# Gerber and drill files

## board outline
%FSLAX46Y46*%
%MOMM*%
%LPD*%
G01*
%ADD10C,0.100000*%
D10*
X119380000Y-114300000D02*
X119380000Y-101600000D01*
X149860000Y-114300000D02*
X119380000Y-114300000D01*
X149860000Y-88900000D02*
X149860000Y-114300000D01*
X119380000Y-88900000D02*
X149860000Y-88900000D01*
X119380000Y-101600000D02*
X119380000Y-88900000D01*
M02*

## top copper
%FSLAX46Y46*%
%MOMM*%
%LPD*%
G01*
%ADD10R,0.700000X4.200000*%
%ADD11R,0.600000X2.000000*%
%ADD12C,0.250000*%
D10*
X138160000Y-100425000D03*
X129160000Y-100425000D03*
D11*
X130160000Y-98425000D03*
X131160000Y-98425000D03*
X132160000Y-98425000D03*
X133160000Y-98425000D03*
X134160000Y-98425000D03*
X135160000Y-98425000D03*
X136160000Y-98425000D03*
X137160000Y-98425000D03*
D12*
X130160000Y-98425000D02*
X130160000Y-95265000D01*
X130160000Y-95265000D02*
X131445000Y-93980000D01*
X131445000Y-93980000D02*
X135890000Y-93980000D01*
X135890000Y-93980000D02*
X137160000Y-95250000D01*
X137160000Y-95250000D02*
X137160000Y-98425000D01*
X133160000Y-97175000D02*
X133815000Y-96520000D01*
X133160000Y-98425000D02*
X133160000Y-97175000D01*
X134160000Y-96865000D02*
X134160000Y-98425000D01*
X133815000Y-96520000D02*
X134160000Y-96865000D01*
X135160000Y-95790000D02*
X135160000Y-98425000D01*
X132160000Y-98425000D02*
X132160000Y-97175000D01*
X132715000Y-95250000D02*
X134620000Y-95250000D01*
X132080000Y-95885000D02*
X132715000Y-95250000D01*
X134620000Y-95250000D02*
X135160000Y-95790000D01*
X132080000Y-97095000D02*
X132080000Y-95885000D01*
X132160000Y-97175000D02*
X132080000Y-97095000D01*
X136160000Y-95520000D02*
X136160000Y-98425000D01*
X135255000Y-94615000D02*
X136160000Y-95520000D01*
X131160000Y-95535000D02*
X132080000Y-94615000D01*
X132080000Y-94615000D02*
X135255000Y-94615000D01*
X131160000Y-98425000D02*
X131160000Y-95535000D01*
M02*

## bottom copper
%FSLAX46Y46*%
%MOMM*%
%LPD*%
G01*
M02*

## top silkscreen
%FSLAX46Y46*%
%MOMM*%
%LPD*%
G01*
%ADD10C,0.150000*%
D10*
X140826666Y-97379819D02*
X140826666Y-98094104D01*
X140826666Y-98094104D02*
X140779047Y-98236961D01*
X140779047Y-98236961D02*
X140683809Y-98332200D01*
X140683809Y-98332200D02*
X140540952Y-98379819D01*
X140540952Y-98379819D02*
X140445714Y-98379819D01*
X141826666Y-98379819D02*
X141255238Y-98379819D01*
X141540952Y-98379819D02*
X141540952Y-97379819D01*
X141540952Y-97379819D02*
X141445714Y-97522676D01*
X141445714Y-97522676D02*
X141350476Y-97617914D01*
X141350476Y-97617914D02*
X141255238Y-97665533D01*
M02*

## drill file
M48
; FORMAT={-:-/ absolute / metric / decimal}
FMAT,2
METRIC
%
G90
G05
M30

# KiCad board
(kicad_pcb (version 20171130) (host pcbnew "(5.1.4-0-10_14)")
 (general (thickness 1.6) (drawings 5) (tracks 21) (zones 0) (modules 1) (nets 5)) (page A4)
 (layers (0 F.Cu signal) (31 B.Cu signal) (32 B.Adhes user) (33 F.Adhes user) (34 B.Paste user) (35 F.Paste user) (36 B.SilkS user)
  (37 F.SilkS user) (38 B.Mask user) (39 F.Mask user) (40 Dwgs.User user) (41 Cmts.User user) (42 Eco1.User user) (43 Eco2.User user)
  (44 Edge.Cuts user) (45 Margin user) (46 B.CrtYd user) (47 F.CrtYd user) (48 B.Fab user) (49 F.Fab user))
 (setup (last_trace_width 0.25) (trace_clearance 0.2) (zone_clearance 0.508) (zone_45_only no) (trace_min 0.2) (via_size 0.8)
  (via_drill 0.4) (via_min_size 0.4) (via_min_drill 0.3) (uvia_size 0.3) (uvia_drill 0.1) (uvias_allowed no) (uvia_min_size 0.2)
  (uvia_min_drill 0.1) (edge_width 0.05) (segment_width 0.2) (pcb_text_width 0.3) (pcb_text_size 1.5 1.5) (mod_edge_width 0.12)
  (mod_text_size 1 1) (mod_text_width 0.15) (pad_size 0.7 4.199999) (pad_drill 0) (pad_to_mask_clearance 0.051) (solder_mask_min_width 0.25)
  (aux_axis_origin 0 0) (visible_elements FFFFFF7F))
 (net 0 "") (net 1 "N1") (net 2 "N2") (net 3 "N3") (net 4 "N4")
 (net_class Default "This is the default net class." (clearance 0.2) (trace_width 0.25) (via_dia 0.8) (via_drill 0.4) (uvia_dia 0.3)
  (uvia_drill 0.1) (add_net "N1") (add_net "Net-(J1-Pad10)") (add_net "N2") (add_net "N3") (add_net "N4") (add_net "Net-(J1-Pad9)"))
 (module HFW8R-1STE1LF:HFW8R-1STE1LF (layer F.Cu) (at 137.16 98.425)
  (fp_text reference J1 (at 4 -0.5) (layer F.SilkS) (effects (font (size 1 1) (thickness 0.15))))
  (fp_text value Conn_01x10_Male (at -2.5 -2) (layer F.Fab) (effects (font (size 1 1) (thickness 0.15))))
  (pad 10 smd rect (at 1 2) (size 0.7 4.2) (layers F.Cu F.Paste F.Mask))
  (pad 9 smd rect (at -8 2) (size 0.7 4.2) (layers F.Cu F.Paste F.Mask))
  (pad 8 smd rect (at -7 0) (size 0.6 2) (layers F.Cu F.Paste F.Mask) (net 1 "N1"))
  (pad 7 smd rect (at -6 0) (size 0.6 2) (layers F.Cu F.Paste F.Mask) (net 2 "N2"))
  (pad 6 smd rect (at -5 0) (size 0.6 2) (layers F.Cu F.Paste F.Mask) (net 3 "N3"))
  (pad 5 smd rect (at -4 0) (size 0.6 2) (layers F.Cu F.Paste F.Mask) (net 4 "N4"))
  (pad 4 smd rect (at -3 0) (size 0.6 2) (layers F.Cu F.Paste F.Mask) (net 4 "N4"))
  (pad 3 smd rect (at -2 0) (size 0.6 2) (layers F.Cu F.Paste F.Mask) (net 3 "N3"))
  (pad 2 smd rect (at -1 0) (size 0.6 2) (layers F.Cu F.Paste F.Mask) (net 2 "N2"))
  (pad 1 smd rect (at 0 0) (size 0.6 2) (layers F.Cu F.Paste F.Mask) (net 1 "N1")))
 (gr_line (start 119.38 114.3) (end 119.38 101.6) (layer Edge.Cuts) (width 0.1))
 (gr_line (start 149.86 114.3) (end 119.38 114.3) (layer Edge.Cuts) (width 0.1))
 (gr_line (start 149.86 88.9) (end 149.86 114.3) (layer Edge.Cuts) (width 0.1))
 (gr_line (start 119.38 88.9) (end 149.86 88.9) (layer Edge.Cuts) (width 0.1))
 (gr_line (start 119.38 101.6) (end 119.38 88.9) (layer Edge.Cuts) (width 0.1))
 (segment (start 130.16 98.425) (end 130.16 95.265) (width 0.25) (layer F.Cu) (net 1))
 (segment (start 130.16 95.265) (end 131.445 93.98) (width 0.25) (layer F.Cu) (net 1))
 (segment (start 131.445 93.98) (end 135.89 93.98) (width 0.25) (layer F.Cu) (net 1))
 (segment (start 135.89 93.98) (end 137.16 95.25) (width 0.25) (layer F.Cu) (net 1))
 (segment (start 137.16 95.25) (end 137.16 98.425) (width 0.25) (layer F.Cu) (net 1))
 (segment (start 133.16 97.175) (end 133.815 96.52) (width 0.25) (layer F.Cu) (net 4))
 (segment (start 133.16 98.425) (end 133.16 97.175) (width 0.25) (layer F.Cu) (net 4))
 (segment (start 134.16 96.865) (end 134.16 98.425) (width 0.25) (layer F.Cu) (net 4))
 (segment (start 133.815 96.52) (end 134.16 96.865) (width 0.25) (layer F.Cu) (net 4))
 (segment (start 135.16 95.79) (end 135.16 98.425) (width 0.25) (layer F.Cu) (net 3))
 (segment (start 132.16 98.425) (end 132.16 97.175) (width 0.25) (layer F.Cu) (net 3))
 (segment (start 132.715 95.25) (end 134.62 95.25) (width 0.25) (layer F.Cu) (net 3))
 (segment (start 132.08 95.885) (end 132.715 95.25) (width 0.25) (layer F.Cu) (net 3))
 (segment (start 134.62 95.25) (end 135.16 95.79) (width 0.25) (layer F.Cu) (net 3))
 (segment (start 132.08 97.095) (end 132.08 95.885) (width 0.25) (layer F.Cu) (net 3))
 (segment (start 132.16 97.175) (end 132.08 97.095) (width 0.25) (layer F.Cu) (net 3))
 (segment (start 136.16 95.52) (end 136.16 98.425) (width 0.25) (layer F.Cu) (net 2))
 (segment (start 135.255 94.615) (end 136.16 95.52) (width 0.25) (layer F.Cu) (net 2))
 (segment (start 131.16 95.535) (end 132.08 94.615) (width 0.25) (layer F.Cu) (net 2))
 (segment (start 132.08 94.615) (end 135.255 94.615) (width 0.25) (layer F.Cu) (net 2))
 (segment (start 131.16 98.425) (end 131.16 95.535) (width 0.25) (layer F.Cu) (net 2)))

